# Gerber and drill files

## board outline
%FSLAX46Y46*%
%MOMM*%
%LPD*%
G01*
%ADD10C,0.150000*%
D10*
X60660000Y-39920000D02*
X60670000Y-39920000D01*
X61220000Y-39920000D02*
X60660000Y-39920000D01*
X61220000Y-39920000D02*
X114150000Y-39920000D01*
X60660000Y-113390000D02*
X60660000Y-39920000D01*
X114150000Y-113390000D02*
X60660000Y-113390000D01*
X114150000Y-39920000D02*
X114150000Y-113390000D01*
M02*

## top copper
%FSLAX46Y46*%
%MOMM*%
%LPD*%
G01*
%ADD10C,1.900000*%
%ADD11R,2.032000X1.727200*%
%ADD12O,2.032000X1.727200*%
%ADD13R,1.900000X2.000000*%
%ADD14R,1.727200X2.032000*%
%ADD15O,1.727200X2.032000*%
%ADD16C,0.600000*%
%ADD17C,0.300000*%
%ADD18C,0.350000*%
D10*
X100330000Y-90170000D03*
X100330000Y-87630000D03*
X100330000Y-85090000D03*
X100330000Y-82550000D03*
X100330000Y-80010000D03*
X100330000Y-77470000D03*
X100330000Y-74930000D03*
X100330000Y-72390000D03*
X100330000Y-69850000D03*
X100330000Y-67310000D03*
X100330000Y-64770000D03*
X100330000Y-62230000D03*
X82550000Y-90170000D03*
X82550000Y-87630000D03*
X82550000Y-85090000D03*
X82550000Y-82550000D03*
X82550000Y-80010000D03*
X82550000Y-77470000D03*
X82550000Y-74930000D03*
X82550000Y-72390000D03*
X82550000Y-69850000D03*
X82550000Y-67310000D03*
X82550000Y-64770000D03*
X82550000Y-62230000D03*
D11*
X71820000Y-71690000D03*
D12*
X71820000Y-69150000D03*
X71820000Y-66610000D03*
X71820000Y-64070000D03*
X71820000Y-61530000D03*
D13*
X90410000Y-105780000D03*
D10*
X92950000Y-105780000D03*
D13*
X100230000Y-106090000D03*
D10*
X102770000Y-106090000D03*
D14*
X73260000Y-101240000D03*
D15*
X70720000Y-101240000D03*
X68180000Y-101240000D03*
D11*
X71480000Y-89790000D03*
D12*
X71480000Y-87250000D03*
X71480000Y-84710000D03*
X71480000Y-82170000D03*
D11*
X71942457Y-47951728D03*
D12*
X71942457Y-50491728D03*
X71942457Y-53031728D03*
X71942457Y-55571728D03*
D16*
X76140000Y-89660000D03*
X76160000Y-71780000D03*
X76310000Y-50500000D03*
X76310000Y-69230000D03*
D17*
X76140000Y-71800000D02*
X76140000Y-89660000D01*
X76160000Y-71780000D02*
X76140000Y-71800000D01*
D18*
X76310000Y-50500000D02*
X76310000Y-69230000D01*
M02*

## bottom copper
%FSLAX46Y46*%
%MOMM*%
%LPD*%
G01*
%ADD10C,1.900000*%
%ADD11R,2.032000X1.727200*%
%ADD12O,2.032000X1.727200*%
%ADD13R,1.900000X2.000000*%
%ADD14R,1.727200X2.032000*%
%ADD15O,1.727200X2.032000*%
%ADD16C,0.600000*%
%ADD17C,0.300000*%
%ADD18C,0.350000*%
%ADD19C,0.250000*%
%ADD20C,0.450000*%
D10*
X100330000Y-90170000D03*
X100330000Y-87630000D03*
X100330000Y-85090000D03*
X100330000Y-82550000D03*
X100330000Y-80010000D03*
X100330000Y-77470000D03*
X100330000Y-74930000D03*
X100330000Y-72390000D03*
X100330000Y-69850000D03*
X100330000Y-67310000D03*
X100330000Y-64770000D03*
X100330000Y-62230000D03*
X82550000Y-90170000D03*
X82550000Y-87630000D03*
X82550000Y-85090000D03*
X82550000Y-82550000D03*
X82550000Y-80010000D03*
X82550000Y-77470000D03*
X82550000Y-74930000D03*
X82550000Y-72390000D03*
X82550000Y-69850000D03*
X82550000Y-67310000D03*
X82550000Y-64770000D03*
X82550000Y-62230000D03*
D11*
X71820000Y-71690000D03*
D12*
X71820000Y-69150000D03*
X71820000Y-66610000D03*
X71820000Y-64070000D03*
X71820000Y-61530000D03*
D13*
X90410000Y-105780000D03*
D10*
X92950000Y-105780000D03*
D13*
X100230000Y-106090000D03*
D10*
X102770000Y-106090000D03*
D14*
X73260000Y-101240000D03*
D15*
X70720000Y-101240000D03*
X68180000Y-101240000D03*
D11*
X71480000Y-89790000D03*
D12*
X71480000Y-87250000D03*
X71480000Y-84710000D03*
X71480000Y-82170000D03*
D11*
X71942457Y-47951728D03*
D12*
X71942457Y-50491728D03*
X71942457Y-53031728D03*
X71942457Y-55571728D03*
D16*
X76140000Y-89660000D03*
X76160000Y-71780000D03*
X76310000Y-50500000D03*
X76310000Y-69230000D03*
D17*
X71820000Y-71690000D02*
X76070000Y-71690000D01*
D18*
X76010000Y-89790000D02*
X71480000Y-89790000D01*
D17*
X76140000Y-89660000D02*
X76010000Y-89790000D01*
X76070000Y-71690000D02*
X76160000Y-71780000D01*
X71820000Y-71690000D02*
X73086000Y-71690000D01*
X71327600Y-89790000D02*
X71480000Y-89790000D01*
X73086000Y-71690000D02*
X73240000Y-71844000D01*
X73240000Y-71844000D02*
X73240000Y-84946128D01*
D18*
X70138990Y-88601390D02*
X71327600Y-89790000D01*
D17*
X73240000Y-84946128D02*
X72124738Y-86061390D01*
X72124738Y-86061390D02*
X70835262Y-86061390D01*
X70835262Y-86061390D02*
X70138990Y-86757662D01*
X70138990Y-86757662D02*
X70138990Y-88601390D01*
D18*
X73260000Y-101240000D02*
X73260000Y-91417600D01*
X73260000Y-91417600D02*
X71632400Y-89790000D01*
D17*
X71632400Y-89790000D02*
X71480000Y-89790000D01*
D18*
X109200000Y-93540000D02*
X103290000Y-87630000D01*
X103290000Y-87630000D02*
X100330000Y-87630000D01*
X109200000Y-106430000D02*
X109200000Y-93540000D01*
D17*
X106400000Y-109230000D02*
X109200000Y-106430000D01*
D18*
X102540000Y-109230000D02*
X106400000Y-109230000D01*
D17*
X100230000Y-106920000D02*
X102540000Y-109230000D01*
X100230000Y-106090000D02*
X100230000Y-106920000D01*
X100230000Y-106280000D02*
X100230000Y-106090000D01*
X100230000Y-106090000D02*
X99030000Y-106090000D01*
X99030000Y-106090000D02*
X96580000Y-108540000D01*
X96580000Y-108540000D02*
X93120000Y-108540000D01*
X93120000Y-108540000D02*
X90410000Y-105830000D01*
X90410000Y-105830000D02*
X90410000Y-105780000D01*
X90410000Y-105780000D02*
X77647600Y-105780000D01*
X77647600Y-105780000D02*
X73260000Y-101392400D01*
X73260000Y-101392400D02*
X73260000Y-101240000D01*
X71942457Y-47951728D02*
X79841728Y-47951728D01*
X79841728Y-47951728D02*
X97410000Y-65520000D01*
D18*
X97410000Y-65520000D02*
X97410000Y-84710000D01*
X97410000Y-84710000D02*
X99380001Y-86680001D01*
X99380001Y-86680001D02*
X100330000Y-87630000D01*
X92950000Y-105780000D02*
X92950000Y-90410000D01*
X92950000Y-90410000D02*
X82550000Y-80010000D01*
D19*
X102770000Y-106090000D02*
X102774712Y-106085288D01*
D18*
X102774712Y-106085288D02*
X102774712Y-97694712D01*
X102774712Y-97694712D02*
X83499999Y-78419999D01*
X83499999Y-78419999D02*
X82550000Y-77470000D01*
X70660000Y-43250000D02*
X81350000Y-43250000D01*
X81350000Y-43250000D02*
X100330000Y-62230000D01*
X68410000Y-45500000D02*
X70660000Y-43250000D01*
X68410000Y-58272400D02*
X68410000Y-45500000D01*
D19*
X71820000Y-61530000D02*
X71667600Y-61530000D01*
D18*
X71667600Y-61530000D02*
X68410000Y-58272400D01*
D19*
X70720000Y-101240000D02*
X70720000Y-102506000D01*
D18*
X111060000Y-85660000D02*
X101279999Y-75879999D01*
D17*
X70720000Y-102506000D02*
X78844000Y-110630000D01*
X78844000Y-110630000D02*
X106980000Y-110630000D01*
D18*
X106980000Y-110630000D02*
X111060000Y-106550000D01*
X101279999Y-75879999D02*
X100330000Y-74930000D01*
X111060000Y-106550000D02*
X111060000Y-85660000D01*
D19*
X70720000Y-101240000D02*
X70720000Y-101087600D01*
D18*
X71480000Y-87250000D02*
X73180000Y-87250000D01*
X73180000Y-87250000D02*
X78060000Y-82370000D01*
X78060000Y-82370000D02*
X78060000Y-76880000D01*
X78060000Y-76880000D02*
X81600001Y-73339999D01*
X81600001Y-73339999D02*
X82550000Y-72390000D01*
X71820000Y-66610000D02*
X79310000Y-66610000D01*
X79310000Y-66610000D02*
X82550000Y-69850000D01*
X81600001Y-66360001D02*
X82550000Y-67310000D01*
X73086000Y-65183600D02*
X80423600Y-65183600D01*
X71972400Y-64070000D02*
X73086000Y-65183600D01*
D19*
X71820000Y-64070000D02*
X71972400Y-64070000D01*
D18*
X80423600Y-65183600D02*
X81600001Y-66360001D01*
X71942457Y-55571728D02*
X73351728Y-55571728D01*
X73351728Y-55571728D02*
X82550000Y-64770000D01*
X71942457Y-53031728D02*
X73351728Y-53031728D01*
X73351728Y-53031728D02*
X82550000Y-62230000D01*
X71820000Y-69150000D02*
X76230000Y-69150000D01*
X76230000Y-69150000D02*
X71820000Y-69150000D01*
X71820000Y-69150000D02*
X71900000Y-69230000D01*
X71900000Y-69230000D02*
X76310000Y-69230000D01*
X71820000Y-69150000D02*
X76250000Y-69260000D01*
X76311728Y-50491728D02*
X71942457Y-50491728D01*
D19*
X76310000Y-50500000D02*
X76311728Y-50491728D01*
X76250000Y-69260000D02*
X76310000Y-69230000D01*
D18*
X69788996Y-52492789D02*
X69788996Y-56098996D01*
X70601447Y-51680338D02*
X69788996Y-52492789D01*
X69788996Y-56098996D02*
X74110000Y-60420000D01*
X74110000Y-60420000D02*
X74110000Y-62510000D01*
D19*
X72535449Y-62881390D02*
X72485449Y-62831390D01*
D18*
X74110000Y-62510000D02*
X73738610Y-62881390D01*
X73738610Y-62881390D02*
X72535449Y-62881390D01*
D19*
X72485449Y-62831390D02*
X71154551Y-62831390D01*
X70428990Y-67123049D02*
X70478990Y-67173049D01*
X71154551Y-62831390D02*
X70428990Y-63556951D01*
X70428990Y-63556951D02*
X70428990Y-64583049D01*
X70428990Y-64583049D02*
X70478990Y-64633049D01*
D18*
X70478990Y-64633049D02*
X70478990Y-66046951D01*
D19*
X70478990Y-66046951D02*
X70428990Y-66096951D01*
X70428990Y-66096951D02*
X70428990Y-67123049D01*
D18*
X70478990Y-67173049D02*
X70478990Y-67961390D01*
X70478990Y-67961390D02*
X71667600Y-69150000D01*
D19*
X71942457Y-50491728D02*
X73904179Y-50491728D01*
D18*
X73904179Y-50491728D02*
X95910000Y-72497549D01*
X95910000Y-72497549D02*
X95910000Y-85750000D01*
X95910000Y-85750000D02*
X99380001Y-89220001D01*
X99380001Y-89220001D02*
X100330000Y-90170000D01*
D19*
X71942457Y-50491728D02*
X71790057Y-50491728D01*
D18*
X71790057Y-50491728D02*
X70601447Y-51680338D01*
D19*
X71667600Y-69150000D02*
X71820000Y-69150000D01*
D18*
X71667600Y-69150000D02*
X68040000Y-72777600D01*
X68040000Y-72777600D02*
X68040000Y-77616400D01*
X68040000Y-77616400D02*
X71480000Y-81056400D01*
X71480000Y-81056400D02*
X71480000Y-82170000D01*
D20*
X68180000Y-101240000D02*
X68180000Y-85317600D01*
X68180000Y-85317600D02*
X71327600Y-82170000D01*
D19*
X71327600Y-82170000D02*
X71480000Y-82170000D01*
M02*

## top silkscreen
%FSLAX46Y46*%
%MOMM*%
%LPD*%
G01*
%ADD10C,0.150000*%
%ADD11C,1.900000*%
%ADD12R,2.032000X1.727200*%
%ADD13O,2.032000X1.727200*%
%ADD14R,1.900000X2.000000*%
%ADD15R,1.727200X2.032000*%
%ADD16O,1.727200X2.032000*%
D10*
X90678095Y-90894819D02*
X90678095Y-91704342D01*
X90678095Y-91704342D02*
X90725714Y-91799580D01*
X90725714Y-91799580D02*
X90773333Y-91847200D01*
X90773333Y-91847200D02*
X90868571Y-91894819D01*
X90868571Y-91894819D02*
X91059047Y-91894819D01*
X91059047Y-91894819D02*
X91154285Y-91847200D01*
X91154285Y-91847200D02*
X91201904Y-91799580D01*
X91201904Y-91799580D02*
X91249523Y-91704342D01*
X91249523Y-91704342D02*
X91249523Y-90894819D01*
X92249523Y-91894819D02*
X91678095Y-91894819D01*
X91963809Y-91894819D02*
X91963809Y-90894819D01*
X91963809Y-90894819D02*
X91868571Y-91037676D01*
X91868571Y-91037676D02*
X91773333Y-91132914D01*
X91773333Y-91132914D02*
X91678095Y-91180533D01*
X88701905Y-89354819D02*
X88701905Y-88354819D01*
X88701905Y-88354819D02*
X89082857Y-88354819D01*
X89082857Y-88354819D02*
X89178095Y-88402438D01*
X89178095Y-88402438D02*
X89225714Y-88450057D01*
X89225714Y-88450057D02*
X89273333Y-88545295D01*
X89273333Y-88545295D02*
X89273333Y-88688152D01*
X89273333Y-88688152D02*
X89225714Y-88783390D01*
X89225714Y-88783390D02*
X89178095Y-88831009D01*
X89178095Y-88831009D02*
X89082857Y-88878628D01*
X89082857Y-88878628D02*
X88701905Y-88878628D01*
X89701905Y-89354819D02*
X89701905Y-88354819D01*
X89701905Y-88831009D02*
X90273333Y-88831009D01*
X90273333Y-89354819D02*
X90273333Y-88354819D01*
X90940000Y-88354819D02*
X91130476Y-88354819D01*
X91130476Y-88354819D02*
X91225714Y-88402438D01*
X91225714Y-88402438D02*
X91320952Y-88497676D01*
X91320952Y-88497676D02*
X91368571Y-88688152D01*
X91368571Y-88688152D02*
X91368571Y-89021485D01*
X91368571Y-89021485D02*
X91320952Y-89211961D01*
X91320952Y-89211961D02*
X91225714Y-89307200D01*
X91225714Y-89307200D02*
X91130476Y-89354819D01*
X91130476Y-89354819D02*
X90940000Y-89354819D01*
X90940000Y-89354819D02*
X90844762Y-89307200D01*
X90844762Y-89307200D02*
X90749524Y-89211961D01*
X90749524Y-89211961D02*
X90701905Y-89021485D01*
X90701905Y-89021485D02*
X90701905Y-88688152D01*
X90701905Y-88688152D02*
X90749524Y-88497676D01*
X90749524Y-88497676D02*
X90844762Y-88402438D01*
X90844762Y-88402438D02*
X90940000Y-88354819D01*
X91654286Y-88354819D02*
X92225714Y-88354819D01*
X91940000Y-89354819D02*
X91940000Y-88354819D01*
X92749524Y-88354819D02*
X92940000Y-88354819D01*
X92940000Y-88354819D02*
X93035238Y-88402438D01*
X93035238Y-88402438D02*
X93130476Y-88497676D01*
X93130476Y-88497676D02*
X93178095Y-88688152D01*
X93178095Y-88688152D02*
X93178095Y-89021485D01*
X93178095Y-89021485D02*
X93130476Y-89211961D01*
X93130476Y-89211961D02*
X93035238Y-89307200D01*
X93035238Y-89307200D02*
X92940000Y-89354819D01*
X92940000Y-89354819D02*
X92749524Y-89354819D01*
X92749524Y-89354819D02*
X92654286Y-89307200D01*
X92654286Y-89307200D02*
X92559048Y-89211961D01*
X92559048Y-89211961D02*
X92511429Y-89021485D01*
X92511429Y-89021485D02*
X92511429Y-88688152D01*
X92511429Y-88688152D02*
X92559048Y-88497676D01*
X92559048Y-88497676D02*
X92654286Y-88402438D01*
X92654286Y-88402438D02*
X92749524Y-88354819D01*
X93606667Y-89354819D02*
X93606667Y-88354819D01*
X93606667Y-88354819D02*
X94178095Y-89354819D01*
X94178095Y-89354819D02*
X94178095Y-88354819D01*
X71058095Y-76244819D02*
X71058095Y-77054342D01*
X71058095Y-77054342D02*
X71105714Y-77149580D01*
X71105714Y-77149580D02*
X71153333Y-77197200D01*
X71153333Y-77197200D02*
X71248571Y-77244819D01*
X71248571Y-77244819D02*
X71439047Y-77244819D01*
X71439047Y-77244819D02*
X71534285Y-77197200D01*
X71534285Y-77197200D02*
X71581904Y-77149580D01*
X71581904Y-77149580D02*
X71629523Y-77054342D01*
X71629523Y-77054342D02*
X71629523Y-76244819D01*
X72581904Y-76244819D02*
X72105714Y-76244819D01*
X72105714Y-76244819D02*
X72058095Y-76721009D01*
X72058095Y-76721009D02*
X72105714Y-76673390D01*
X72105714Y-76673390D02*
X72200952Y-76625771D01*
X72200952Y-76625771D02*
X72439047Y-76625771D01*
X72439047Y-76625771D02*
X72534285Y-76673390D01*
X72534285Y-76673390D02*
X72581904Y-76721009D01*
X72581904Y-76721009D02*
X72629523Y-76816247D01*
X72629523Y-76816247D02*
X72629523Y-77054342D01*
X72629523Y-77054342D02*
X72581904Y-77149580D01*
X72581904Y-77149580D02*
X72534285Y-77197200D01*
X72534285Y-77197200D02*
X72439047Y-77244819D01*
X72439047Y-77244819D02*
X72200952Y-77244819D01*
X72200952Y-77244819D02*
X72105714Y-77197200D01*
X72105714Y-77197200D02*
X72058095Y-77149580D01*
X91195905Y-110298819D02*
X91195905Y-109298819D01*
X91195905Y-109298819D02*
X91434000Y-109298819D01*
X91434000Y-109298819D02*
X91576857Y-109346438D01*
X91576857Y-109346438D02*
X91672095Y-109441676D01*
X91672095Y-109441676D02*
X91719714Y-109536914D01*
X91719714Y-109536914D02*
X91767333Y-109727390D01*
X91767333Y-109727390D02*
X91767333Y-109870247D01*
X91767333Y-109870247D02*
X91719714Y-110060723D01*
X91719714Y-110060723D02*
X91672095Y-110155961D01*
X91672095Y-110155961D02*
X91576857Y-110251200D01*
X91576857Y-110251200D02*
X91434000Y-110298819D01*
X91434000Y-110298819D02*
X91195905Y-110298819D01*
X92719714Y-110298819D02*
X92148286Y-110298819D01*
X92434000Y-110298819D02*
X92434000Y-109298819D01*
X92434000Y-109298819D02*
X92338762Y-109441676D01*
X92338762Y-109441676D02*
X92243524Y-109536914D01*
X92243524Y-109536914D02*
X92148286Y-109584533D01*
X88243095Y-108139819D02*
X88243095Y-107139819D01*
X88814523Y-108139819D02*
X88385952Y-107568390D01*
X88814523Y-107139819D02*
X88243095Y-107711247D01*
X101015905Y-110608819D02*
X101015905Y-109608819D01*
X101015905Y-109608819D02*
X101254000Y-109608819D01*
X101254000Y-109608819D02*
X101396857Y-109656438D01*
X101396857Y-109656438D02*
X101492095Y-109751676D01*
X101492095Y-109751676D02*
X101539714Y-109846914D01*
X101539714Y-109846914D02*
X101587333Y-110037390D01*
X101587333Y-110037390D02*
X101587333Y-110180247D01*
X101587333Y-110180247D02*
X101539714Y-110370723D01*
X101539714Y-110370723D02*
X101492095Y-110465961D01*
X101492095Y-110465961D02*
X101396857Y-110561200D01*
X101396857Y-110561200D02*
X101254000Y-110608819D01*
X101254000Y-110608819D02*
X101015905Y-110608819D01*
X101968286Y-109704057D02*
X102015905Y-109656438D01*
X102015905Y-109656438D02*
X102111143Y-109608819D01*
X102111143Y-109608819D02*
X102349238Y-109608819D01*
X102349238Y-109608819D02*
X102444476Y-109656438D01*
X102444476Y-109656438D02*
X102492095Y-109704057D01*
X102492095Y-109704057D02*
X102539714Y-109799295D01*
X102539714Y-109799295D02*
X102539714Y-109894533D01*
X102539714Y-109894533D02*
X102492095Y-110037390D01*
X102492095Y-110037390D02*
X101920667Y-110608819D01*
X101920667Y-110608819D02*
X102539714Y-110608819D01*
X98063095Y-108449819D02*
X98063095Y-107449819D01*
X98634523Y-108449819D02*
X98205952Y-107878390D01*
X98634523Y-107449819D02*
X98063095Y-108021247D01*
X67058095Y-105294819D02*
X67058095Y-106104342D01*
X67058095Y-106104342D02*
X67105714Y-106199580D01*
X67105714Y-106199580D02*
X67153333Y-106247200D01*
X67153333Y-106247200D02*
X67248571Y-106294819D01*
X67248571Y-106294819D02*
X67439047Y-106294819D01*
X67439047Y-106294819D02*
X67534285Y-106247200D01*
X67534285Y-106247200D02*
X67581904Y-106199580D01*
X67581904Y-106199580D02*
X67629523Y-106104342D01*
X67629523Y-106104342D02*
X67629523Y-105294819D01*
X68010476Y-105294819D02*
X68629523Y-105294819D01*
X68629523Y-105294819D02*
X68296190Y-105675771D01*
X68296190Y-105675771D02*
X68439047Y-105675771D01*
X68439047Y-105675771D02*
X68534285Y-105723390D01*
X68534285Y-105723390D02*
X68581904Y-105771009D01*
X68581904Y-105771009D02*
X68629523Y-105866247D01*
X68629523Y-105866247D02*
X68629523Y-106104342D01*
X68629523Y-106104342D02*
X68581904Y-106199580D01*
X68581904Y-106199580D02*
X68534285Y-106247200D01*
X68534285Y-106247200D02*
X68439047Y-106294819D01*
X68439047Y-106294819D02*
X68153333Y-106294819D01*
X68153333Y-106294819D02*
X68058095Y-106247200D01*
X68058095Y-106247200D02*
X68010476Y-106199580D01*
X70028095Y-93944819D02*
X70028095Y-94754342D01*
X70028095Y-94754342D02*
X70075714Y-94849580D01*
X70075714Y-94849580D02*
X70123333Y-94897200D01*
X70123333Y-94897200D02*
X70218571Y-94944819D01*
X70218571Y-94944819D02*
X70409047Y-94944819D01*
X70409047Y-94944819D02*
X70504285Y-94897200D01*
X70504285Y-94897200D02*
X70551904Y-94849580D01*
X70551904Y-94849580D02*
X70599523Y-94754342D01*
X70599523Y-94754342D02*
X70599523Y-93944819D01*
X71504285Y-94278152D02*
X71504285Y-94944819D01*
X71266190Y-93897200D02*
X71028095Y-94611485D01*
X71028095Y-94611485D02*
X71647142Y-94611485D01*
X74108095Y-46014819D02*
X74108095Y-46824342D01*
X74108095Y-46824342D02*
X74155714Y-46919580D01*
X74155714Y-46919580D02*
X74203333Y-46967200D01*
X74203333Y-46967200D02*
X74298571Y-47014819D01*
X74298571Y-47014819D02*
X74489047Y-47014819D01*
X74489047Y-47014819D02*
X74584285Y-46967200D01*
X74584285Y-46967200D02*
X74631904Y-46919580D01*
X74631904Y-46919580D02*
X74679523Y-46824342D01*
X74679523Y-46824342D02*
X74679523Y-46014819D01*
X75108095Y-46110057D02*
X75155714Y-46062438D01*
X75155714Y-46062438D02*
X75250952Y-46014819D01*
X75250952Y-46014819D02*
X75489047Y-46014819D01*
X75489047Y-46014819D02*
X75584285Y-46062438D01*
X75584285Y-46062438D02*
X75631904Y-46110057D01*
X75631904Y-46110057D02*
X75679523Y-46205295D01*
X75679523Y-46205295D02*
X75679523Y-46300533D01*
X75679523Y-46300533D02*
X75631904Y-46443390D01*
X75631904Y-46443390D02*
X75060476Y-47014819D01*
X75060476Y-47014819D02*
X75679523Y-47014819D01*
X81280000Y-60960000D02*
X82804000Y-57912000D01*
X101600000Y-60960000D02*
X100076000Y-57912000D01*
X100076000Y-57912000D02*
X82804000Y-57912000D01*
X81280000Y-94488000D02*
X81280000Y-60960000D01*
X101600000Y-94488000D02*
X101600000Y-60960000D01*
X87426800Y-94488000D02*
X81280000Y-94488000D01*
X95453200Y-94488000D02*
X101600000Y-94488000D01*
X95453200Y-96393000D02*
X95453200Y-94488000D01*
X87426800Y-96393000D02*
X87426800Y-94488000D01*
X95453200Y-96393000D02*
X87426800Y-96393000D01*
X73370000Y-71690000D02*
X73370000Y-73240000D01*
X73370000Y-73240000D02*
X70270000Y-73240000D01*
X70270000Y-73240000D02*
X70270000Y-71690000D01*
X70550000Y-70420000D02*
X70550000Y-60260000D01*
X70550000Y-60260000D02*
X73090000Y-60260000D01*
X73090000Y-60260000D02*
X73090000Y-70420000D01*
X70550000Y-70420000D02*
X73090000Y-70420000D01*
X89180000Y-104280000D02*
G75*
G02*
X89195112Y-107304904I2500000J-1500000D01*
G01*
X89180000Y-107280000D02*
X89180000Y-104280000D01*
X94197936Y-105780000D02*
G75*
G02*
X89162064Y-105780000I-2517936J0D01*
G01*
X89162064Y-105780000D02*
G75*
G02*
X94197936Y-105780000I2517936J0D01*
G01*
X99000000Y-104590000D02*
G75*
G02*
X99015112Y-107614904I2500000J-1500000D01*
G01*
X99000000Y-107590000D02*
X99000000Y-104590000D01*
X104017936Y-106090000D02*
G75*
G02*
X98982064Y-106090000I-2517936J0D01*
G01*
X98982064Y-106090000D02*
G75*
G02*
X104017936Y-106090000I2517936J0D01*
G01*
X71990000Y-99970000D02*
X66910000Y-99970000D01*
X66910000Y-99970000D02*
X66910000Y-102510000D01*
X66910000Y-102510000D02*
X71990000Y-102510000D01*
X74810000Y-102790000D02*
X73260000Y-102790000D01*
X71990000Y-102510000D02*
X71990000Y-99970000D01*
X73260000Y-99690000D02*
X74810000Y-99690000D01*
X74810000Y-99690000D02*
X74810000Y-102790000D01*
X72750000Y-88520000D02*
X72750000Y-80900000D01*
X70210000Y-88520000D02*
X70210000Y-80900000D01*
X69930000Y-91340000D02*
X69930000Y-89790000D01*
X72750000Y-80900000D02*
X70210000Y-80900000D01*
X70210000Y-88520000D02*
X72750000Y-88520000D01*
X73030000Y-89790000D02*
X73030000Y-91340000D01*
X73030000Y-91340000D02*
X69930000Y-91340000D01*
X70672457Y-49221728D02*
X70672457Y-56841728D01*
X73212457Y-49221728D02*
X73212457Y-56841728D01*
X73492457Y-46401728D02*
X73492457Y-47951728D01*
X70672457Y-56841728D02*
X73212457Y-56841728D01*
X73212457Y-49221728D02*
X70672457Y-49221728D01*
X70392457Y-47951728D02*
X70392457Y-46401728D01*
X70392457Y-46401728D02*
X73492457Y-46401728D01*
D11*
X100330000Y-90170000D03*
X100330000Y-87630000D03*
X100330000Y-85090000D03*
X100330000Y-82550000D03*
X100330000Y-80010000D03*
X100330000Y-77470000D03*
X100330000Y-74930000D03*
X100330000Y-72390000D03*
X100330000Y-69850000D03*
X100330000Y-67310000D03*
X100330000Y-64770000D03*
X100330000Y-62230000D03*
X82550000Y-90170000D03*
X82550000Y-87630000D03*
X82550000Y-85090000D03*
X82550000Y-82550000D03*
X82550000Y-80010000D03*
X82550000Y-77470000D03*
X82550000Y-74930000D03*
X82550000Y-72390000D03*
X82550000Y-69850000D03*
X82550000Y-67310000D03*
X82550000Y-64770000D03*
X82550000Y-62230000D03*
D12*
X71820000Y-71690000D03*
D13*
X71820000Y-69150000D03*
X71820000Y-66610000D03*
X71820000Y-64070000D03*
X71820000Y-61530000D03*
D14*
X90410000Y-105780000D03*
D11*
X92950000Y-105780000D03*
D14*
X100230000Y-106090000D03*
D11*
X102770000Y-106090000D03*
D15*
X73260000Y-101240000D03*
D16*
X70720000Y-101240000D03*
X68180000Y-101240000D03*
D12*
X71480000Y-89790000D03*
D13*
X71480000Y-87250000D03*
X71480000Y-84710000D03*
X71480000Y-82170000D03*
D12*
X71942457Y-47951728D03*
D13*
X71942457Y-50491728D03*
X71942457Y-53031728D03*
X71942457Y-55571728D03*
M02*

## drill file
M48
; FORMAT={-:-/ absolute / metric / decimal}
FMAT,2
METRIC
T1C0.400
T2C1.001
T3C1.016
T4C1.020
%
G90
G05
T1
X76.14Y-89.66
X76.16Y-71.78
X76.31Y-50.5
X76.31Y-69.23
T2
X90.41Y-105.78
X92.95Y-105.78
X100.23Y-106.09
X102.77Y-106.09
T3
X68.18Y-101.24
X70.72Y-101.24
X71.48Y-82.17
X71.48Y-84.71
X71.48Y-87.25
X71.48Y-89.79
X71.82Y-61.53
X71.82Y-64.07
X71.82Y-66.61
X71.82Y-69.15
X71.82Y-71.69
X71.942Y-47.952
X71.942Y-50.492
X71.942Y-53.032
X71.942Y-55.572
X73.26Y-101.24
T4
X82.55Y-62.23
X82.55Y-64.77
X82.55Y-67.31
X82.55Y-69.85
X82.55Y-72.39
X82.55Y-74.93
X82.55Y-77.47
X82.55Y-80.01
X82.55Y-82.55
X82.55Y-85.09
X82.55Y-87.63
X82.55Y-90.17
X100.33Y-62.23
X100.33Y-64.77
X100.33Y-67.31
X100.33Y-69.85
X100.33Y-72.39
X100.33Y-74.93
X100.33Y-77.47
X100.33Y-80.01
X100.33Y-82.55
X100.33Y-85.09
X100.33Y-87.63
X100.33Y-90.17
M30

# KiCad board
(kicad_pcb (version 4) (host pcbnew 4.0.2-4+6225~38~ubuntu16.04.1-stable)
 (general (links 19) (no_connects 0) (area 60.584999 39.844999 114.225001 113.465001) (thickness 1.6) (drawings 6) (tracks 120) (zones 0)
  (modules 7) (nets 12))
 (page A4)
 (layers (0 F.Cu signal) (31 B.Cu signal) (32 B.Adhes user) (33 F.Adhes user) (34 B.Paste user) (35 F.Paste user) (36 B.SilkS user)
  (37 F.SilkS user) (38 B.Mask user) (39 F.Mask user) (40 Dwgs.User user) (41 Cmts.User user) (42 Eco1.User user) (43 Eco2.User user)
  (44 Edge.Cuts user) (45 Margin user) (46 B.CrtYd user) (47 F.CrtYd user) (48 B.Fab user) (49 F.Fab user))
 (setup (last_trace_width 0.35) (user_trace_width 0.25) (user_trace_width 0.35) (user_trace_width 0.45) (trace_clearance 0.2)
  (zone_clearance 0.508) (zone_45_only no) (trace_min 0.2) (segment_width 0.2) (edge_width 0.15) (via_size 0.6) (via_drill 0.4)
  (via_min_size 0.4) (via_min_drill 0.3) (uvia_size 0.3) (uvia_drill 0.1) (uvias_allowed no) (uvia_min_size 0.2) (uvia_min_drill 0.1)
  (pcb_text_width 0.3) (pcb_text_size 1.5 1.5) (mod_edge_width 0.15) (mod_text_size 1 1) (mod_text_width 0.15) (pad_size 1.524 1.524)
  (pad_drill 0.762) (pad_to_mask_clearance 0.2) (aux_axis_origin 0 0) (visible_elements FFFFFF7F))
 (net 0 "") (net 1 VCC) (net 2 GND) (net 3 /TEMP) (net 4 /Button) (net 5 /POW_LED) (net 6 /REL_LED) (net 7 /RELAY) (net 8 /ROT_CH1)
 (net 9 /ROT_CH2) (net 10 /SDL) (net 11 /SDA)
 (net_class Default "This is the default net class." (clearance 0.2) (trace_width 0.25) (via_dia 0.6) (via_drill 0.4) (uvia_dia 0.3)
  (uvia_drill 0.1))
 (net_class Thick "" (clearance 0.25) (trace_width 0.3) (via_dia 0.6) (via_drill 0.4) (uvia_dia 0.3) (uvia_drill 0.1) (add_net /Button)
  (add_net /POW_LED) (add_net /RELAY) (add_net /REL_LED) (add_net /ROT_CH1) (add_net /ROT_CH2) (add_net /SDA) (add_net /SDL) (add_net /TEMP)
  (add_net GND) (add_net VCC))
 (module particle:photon (layer F.Cu) (at 91.44 74.93 180)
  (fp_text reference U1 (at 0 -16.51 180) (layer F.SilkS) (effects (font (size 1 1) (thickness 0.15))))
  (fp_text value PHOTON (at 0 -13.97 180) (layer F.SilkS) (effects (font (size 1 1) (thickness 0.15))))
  (fp_line (start 10.16 13.97) (end 8.636 17.018) (layer F.SilkS) (width 0.15))
  (fp_line (start -10.16 13.97) (end -8.636 17.018) (layer F.SilkS) (width 0.15))
  (fp_line (start -8.636 17.018) (end 8.636 17.018) (layer F.SilkS) (width 0.15))
  (fp_line (start 10.16 -19.558) (end 10.16 13.97) (layer F.SilkS) (width 0.15))
  (fp_line (start -10.16 -19.558) (end -10.16 13.97) (layer F.SilkS) (width 0.15))
  (fp_line (start 4.0132 -19.558) (end 10.16 -19.558) (layer F.SilkS) (width 0.15))
  (fp_line (start -4.0132 -19.558) (end -10.16 -19.558) (layer F.SilkS) (width 0.15))
  (fp_line (start -4.0132 -21.463) (end -4.0132 -19.558) (layer F.SilkS) (width 0.15))
  (fp_line (start 4.0132 -21.463) (end 4.0132 -19.558) (layer F.SilkS) (width 0.15))
  (fp_line (start -4.0132 -21.463) (end 4.0132 -21.463) (layer F.SilkS) (width 0.15))
  (pad 1 thru_hole circle (at -8.89 -15.24 180) (size 1.9 1.9) (drill 1.02) (layers *.Cu *.Mask F.SilkS) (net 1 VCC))
  (pad 2 thru_hole circle (at -8.89 -12.7 180) (size 1.9 1.9) (drill 1.02) (layers *.Cu *.Mask F.SilkS) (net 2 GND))
  (pad 3 thru_hole circle (at -8.89 -10.16 180) (size 1.9 1.9) (drill 1.02) (layers *.Cu *.Mask F.SilkS))
  (pad 4 thru_hole circle (at -8.89 -7.62 180) (size 1.9 1.9) (drill 1.02) (layers *.Cu *.Mask F.SilkS))
  (pad 5 thru_hole circle (at -8.89 -5.08 180) (size 1.9 1.9) (drill 1.02) (layers *.Cu *.Mask F.SilkS))
  (pad 6 thru_hole circle (at -8.89 -2.54 180) (size 1.9 1.9) (drill 1.02) (layers *.Cu *.Mask F.SilkS))
  (pad 7 thru_hole circle (at -8.89 0 180) (size 1.9 1.9) (drill 1.02) (layers *.Cu *.Mask F.SilkS) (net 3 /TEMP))
  (pad 8 thru_hole circle (at -8.89 2.54 180) (size 1.9 1.9) (drill 1.02) (layers *.Cu *.Mask F.SilkS))
  (pad 9 thru_hole circle (at -8.89 5.08 180) (size 1.9 1.9) (drill 1.02) (layers *.Cu *.Mask F.SilkS))
  (pad 10 thru_hole circle (at -8.89 7.62 180) (size 1.9 1.9) (drill 1.02) (layers *.Cu *.Mask F.SilkS))
  (pad 11 thru_hole circle (at -8.89 10.16 180) (size 1.9 1.9) (drill 1.02) (layers *.Cu *.Mask F.SilkS))
  (pad 12 thru_hole circle (at -8.89 12.7 180) (size 1.9 1.9) (drill 1.02) (layers *.Cu *.Mask F.SilkS) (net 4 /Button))
  (pad 24 thru_hole circle (at 8.89 -15.24 180) (size 1.9 1.9) (drill 1.02) (layers *.Cu *.Mask F.SilkS))
  (pad 23 thru_hole circle (at 8.89 -12.7 180) (size 1.9 1.9) (drill 1.02) (layers *.Cu *.Mask F.SilkS))
  (pad 22 thru_hole circle (at 8.89 -10.16 180) (size 1.9 1.9) (drill 1.02) (layers *.Cu *.Mask F.SilkS))
  (pad 21 thru_hole circle (at 8.89 -7.62 180) (size 1.9 1.9) (drill 1.02) (layers *.Cu *.Mask F.SilkS))
  (pad 20 thru_hole circle (at 8.89 -5.08 180) (size 1.9 1.9) (drill 1.02) (layers *.Cu *.Mask F.SilkS) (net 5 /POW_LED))
  (pad 19 thru_hole circle (at 8.89 -2.54 180) (size 1.9 1.9) (drill 1.02) (layers *.Cu *.Mask F.SilkS) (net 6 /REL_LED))
  (pad 18 thru_hole circle (at 8.89 0 180) (size 1.9 1.9) (drill 1.02) (layers *.Cu *.Mask F.SilkS))
  (pad 17 thru_hole circle (at 8.89 2.54 180) (size 1.9 1.9) (drill 1.02) (layers *.Cu *.Mask F.SilkS) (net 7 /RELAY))
  (pad 16 thru_hole circle (at 8.89 5.08 180) (size 1.9 1.9) (drill 1.02) (layers *.Cu *.Mask F.SilkS) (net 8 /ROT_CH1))
  (pad 15 thru_hole circle (at 8.89 7.62 180) (size 1.9 1.9) (drill 1.02) (layers *.Cu *.Mask F.SilkS) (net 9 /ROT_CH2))
  (pad 14 thru_hole circle (at 8.89 10.16 180) (size 1.9 1.9) (drill 1.02) (layers *.Cu *.Mask F.SilkS) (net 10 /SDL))
  (pad 13 thru_hole circle (at 8.89 12.7 180) (size 1.9 1.9) (drill 1.02) (layers *.Cu *.Mask F.SilkS) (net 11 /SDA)))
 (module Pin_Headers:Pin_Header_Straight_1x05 (layer F.Cu) (at 71.82 71.69 180)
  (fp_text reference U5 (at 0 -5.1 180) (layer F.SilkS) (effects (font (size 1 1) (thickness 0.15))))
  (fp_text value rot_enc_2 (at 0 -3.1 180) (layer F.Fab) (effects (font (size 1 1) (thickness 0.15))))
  (fp_line (start -1.55 0) (end -1.55 -1.55) (layer F.SilkS) (width 0.15))
  (fp_line (start -1.55 -1.55) (end 1.55 -1.55) (layer F.SilkS) (width 0.15))
  (fp_line (start 1.55 -1.55) (end 1.55 0) (layer F.SilkS) (width 0.15))
  (fp_line (start 1.27 1.27) (end 1.27 11.43) (layer F.SilkS) (width 0.15))
  (fp_line (start 1.27 11.43) (end -1.27 11.43) (layer F.SilkS) (width 0.15))
  (fp_line (start -1.27 11.43) (end -1.27 1.27) (layer F.SilkS) (width 0.15))
  (fp_line (start 1.27 1.27) (end -1.27 1.27) (layer F.SilkS) (width 0.15))
  (pad 1 thru_hole rect (at 0 0 180) (size 2.032 1.7272) (drill 1.016) (layers *.Cu *.Mask F.SilkS) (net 2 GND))
  (pad 2 thru_hole oval (at 0 2.54 180) (size 2.032 1.7272) (drill 1.016) (layers *.Cu *.Mask F.SilkS) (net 1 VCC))
  (pad 3 thru_hole oval (at 0 5.08 180) (size 2.032 1.7272) (drill 1.016) (layers *.Cu *.Mask F.SilkS) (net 8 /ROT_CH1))
  (pad 4 thru_hole oval (at 0 7.62 180) (size 2.032 1.7272) (drill 1.016) (layers *.Cu *.Mask F.SilkS) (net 9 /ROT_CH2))
  (pad 5 thru_hole oval (at 0 10.16 180) (size 2.032 1.7272) (drill 1.016) (layers *.Cu *.Mask F.SilkS) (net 4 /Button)))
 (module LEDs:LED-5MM (layer F.Cu) (at 90.41 105.78)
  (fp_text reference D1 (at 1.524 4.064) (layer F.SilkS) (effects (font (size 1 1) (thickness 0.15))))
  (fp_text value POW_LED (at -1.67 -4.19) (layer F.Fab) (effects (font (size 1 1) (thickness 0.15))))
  (fp_arc (start 1.27 0) (end -1.23 -1.5) (angle 297.5) (layer F.SilkS) (width 0.15))
  (fp_line (start -1.23 1.5) (end -1.23 -1.5) (layer F.SilkS) (width 0.15))
  (fp_circle (center 1.27 0) (end 0.97 -2.5) (layer F.SilkS) (width 0.15))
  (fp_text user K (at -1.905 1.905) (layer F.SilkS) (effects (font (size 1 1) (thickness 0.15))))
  (pad 1 thru_hole rect (at 0 0 90) (size 2 1.9) (drill 1.00076) (layers *.Cu *.Mask F.SilkS) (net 2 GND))
  (pad 2 thru_hole circle (at 2.54 0) (size 1.9 1.9) (drill 1.00076) (layers *.Cu *.Mask F.SilkS) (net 5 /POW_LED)))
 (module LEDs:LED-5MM (layer F.Cu) (at 100.23 106.09)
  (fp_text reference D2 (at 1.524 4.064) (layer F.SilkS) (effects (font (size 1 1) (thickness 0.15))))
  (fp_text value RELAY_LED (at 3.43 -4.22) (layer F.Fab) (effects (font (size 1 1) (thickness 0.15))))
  (fp_arc (start 1.27 0) (end -1.23 -1.5) (angle 297.5) (layer F.SilkS) (width 0.15))
  (fp_line (start -1.23 1.5) (end -1.23 -1.5) (layer F.SilkS) (width 0.15))
  (fp_circle (center 1.27 0) (end 0.97 -2.5) (layer F.SilkS) (width 0.15))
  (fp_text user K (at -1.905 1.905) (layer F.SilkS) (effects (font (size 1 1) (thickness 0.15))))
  (pad 1 thru_hole rect (at 0 0 90) (size 2 1.9) (drill 1.00076) (layers *.Cu *.Mask F.SilkS) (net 2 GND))
  (pad 2 thru_hole circle (at 2.54 0) (size 1.9 1.9) (drill 1.00076) (layers *.Cu *.Mask F.SilkS) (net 6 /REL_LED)))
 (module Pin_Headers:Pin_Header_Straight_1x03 (layer F.Cu) (at 73.26 101.24 270)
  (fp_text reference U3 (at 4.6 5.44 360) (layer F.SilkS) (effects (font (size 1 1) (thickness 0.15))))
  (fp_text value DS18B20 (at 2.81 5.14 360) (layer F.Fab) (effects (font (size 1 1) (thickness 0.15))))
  (fp_line (start -1.27 1.27) (end -1.27 6.35) (layer F.SilkS) (width 0.15))
  (fp_line (start -1.27 6.35) (end 1.27 6.35) (layer F.SilkS) (width 0.15))
  (fp_line (start 1.27 6.35) (end 1.27 1.27) (layer F.SilkS) (width 0.15))
  (fp_line (start 1.55 -1.55) (end 1.55 0) (layer F.SilkS) (width 0.15))
  (fp_line (start 1.27 1.27) (end -1.27 1.27) (layer F.SilkS) (width 0.15))
  (fp_line (start -1.55 0) (end -1.55 -1.55) (layer F.SilkS) (width 0.15))
  (fp_line (start -1.55 -1.55) (end 1.55 -1.55) (layer F.SilkS) (width 0.15))
  (pad 1 thru_hole rect (at 0 0 270) (size 2.032 1.7272) (drill 1.016) (layers *.Cu *.Mask F.SilkS) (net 2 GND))
  (pad 2 thru_hole oval (at 0 2.54 270) (size 2.032 1.7272) (drill 1.016) (layers *.Cu *.Mask F.SilkS) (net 3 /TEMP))
  (pad 3 thru_hole oval (at 0 5.08 270) (size 2.032 1.7272) (drill 1.016) (layers *.Cu *.Mask F.SilkS) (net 1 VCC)))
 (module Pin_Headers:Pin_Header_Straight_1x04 (layer F.Cu) (at 71.48 89.79 180)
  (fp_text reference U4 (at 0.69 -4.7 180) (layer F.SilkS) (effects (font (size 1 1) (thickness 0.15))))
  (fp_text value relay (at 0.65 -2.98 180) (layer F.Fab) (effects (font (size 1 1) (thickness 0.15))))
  (fp_line (start -1.27 1.27) (end -1.27 8.89) (layer F.SilkS) (width 0.15))
  (fp_line (start 1.27 1.27) (end 1.27 8.89) (layer F.SilkS) (width 0.15))
  (fp_line (start 1.55 -1.55) (end 1.55 0) (layer F.SilkS) (width 0.15))
  (fp_line (start -1.27 8.89) (end 1.27 8.89) (layer F.SilkS) (width 0.15))
  (fp_line (start 1.27 1.27) (end -1.27 1.27) (layer F.SilkS) (width 0.15))
  (fp_line (start -1.55 0) (end -1.55 -1.55) (layer F.SilkS) (width 0.15))
  (fp_line (start -1.55 -1.55) (end 1.55 -1.55) (layer F.SilkS) (width 0.15))
  (pad 1 thru_hole rect (at 0 0 180) (size 2.032 1.7272) (drill 1.016) (layers *.Cu *.Mask F.SilkS) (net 2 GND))
  (pad 2 thru_hole oval (at 0 2.54 180) (size 2.032 1.7272) (drill 1.016) (layers *.Cu *.Mask F.SilkS) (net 7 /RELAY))
  (pad 3 thru_hole oval (at 0 5.08 180) (size 2.032 1.7272) (drill 1.016) (layers *.Cu *.Mask F.SilkS))
  (pad 4 thru_hole oval (at 0 7.62 180) (size 2.032 1.7272) (drill 1.016) (layers *.Cu *.Mask F.SilkS) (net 1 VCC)))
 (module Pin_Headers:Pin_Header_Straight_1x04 (layer F.Cu) (at 71.942457 47.951728)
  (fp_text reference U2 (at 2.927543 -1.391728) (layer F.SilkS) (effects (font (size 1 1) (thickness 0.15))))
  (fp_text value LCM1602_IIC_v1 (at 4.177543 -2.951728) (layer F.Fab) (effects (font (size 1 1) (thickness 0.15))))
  (fp_line (start -1.27 1.27) (end -1.27 8.89) (layer F.SilkS) (width 0.15))
  (fp_line (start 1.27 1.27) (end 1.27 8.89) (layer F.SilkS) (width 0.15))
  (fp_line (start 1.55 -1.55) (end 1.55 0) (layer F.SilkS) (width 0.15))
  (fp_line (start -1.27 8.89) (end 1.27 8.89) (layer F.SilkS) (width 0.15))
  (fp_line (start 1.27 1.27) (end -1.27 1.27) (layer F.SilkS) (width 0.15))
  (fp_line (start -1.55 0) (end -1.55 -1.55) (layer F.SilkS) (width 0.15))
  (fp_line (start -1.55 -1.55) (end 1.55 -1.55) (layer F.SilkS) (width 0.15))
  (pad 1 thru_hole rect (at 0 0) (size 2.032 1.7272) (drill 1.016) (layers *.Cu *.Mask F.SilkS) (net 2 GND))
  (pad 2 thru_hole oval (at 0 2.54) (size 2.032 1.7272) (drill 1.016) (layers *.Cu *.Mask F.SilkS) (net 1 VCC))
  (pad 3 thru_hole oval (at 0 5.08) (size 2.032 1.7272) (drill 1.016) (layers *.Cu *.Mask F.SilkS) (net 11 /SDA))
  (pad 4 thru_hole oval (at 0 7.62) (size 2.032 1.7272) (drill 1.016) (layers *.Cu *.Mask F.SilkS) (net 10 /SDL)))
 (gr_line (start 60.66 39.92) (end 60.67 39.92) (angle 90) (layer Edge.Cuts) (width 0.15))
 (gr_line (start 61.22 39.92) (end 60.66 39.92) (angle 90) (layer Edge.Cuts) (width 0.15))
 (gr_line (start 61.22 39.92) (end 114.15 39.92) (angle 90) (layer Edge.Cuts) (width 0.15))
 (gr_line (start 60.66 113.39) (end 60.66 39.92) (angle 90) (layer Edge.Cuts) (width 0.15))
 (gr_line (start 114.15 113.39) (end 60.66 113.39) (angle 90) (layer Edge.Cuts) (width 0.15))
 (gr_line (start 114.15 39.92) (end 114.15 113.39) (angle 90) (layer Edge.Cuts) (width 0.15))
 (segment (start 71.82 71.69) (end 76.07 71.69) (width 0.3) (layer B.Cu) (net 2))
 (segment (start 76.01 89.79) (end 71.48 89.79) (width 0.35) (layer B.Cu) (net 2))
 (segment (start 76.14 89.66) (end 76.01 89.79) (width 0.3) (layer B.Cu) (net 2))
 (via (at 76.14 89.66) (size 0.6) (drill 0.4) (layers F.Cu B.Cu) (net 2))
 (segment (start 76.14 71.8) (end 76.14 89.66) (width 0.3) (layer F.Cu) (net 2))
 (segment (start 76.16 71.78) (end 76.14 71.8) (width 0.3) (layer F.Cu) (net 2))
 (via (at 76.16 71.78) (size 0.6) (drill 0.4) (layers F.Cu B.Cu) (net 2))
 (segment (start 76.07 71.69) (end 76.16 71.78) (width 0.3) (layer B.Cu) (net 2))
 (segment (start 71.82 71.69) (end 73.086 71.69) (width 0.3) (layer B.Cu) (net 2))
 (segment (start 71.3276 89.79) (end 71.48 89.79) (width 0.3) (layer B.Cu) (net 2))
 (segment (start 73.086 71.69) (end 73.24 71.844) (width 0.3) (layer B.Cu) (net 2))
 (segment (start 73.24 71.844) (end 73.24 84.946128) (width 0.3) (layer B.Cu) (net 2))
 (segment (start 70.13899 88.60139) (end 71.3276 89.79) (width 0.35) (layer B.Cu) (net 2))
 (segment (start 73.24 84.946128) (end 72.124738 86.06139) (width 0.3) (layer B.Cu) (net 2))
 (segment (start 72.124738 86.06139) (end 70.835262 86.06139) (width 0.3) (layer B.Cu) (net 2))
 (segment (start 70.835262 86.06139) (end 70.13899 86.757662) (width 0.3) (layer B.Cu) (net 2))
 (segment (start 70.13899 86.757662) (end 70.13899 88.60139) (width 0.3) (layer B.Cu) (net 2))
 (segment (start 73.26 101.24) (end 73.26 91.4176) (width 0.35) (layer B.Cu) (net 2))
 (segment (start 73.26 91.4176) (end 71.6324 89.79) (width 0.35) (layer B.Cu) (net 2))
 (segment (start 71.6324 89.79) (end 71.48 89.79) (width 0.3) (layer B.Cu) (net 2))
 (segment (start 109.2 93.54) (end 103.29 87.63) (width 0.35) (layer B.Cu) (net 2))
 (segment (start 103.29 87.63) (end 100.33 87.63) (width 0.35) (layer B.Cu) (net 2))
 (segment (start 109.2 106.43) (end 109.2 93.54) (width 0.35) (layer B.Cu) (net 2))
 (segment (start 106.4 109.23) (end 109.2 106.43) (width 0.3) (layer B.Cu) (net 2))
 (segment (start 102.54 109.23) (end 106.4 109.23) (width 0.35) (layer B.Cu) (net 2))
 (segment (start 100.23 106.92) (end 102.54 109.23) (width 0.3) (layer B.Cu) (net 2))
 (segment (start 100.23 106.09) (end 100.23 106.92) (width 0.3) (layer B.Cu) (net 2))
 (segment (start 100.23 106.28) (end 100.23 106.09) (width 0.3) (layer B.Cu) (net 2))
 (segment (start 100.23 106.09) (end 99.03 106.09) (width 0.3) (layer B.Cu) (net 2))
 (segment (start 99.03 106.09) (end 96.58 108.54) (width 0.3) (layer B.Cu) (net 2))
 (segment (start 96.58 108.54) (end 93.12 108.54) (width 0.3) (layer B.Cu) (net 2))
 (segment (start 93.12 108.54) (end 90.41 105.83) (width 0.3) (layer B.Cu) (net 2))
 (segment (start 90.41 105.83) (end 90.41 105.78) (width 0.3) (layer B.Cu) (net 2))
 (segment (start 90.41 105.78) (end 77.6476 105.78) (width 0.3) (layer B.Cu) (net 2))
 (segment (start 77.6476 105.78) (end 73.26 101.3924) (width 0.3) (layer B.Cu) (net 2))
 (segment (start 73.26 101.3924) (end 73.26 101.24) (width 0.3) (layer B.Cu) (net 2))
 (segment (start 71.942457 47.951728) (end 79.841728 47.951728) (width 0.3) (layer B.Cu) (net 2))
 (segment (start 79.841728 47.951728) (end 97.41 65.52) (width 0.3) (layer B.Cu) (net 2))
 (segment (start 97.41 65.52) (end 97.41 84.71) (width 0.35) (layer B.Cu) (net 2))
 (segment (start 97.41 84.71) (end 99.380001 86.680001) (width 0.35) (layer B.Cu) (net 2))
 (segment (start 99.380001 86.680001) (end 100.33 87.63) (width 0.35) (layer B.Cu) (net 2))
 (segment (start 92.95 105.78) (end 92.95 90.41) (width 0.35) (layer B.Cu) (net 5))
 (segment (start 92.95 90.41) (end 82.55 80.01) (width 0.35) (layer B.Cu) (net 5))
 (segment (start 102.77 106.09) (end 102.774712 106.085288) (width 0.25) (layer B.Cu) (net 6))
 (segment (start 102.774712 106.085288) (end 102.774712 97.694712) (width 0.35) (layer B.Cu) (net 6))
 (segment (start 102.774712 97.694712) (end 83.499999 78.419999) (width 0.35) (layer B.Cu) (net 6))
 (segment (start 83.499999 78.419999) (end 82.55 77.47) (width 0.35) (layer B.Cu) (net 6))
 (segment (start 70.66 43.25) (end 81.35 43.25) (width 0.35) (layer B.Cu) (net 4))
 (segment (start 81.35 43.25) (end 100.33 62.23) (width 0.35) (layer B.Cu) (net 4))
 (segment (start 68.41 45.5) (end 70.66 43.25) (width 0.35) (layer B.Cu) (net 4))
 (segment (start 68.41 58.2724) (end 68.41 45.5) (width 0.35) (layer B.Cu) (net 4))
 (segment (start 71.82 61.53) (end 71.6676 61.53) (width 0.25) (layer B.Cu) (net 4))
 (segment (start 71.6676 61.53) (end 68.41 58.2724) (width 0.35) (layer B.Cu) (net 4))
 (segment (start 70.72 101.24) (end 70.72 102.506) (width 0.25) (layer B.Cu) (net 3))
 (segment (start 111.06 85.66) (end 101.279999 75.879999) (width 0.35) (layer B.Cu) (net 3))
 (segment (start 70.72 102.506) (end 78.844 110.63) (width 0.3) (layer B.Cu) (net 3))
 (segment (start 78.844 110.63) (end 106.98 110.63) (width 0.3) (layer B.Cu) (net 3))
 (segment (start 106.98 110.63) (end 111.06 106.55) (width 0.35) (layer B.Cu) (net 3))
 (segment (start 101.279999 75.879999) (end 100.33 74.93) (width 0.35) (layer B.Cu) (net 3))
 (segment (start 111.06 106.55) (end 111.06 85.66) (width 0.35) (layer B.Cu) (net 3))
 (segment (start 70.72 101.24) (end 70.72 101.0876) (width 0.25) (layer B.Cu) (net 3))
 (segment (start 71.48 87.25) (end 73.18 87.25) (width 0.35) (layer B.Cu) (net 7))
 (segment (start 73.18 87.25) (end 78.06 82.37) (width 0.35) (layer B.Cu) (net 7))
 (segment (start 78.06 82.37) (end 78.06 76.88) (width 0.35) (layer B.Cu) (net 7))
 (segment (start 78.06 76.88) (end 81.600001 73.339999) (width 0.35) (layer B.Cu) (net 7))
 (segment (start 81.600001 73.339999) (end 82.55 72.39) (width 0.35) (layer B.Cu) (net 7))
 (segment (start 71.82 66.61) (end 79.31 66.61) (width 0.35) (layer B.Cu) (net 8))
 (segment (start 79.31 66.61) (end 82.55 69.85) (width 0.35) (layer B.Cu) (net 8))
 (segment (start 81.600001 66.360001) (end 82.55 67.31) (width 0.35) (layer B.Cu) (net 9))
 (segment (start 73.086 65.1836) (end 80.4236 65.1836) (width 0.35) (layer B.Cu) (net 9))
 (segment (start 71.9724 64.07) (end 73.086 65.1836) (width 0.35) (layer B.Cu) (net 9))
 (segment (start 71.82 64.07) (end 71.9724 64.07) (width 0.25) (layer B.Cu) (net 9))
 (segment (start 80.4236 65.1836) (end 81.600001 66.360001) (width 0.35) (layer B.Cu) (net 9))
 (segment (start 71.942457 55.571728) (end 73.351728 55.571728) (width 0.35) (layer B.Cu) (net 10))
 (segment (start 73.351728 55.571728) (end 82.55 64.77) (width 0.35) (layer B.Cu) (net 10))
 (segment (start 71.942457 53.031728) (end 73.351728 53.031728) (width 0.35) (layer B.Cu) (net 11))
 (segment (start 73.351728 53.031728) (end 82.55 62.23) (width 0.35) (layer B.Cu) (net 11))
 (segment (start 71.82 69.15) (end 76.23 69.15) (width 0.35) (layer B.Cu) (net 1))
 (segment (start 76.23 69.15) (end 71.82 69.15) (width 0.35) (layer B.Cu) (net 1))
 (segment (start 71.82 69.15) (end 71.9 69.23) (width 0.35) (layer B.Cu) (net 1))
 (segment (start 71.9 69.23) (end 76.31 69.23) (width 0.35) (layer B.Cu) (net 1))
 (segment (start 76.31 50.5) (end 76.31 69.23) (width 0.35) (layer F.Cu) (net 1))
 (segment (start 71.82 69.15) (end 76.25 69.26) (width 0.35) (layer B.Cu) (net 1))
 (segment (start 76.311728 50.491728) (end 71.942457 50.491728) (width 0.35) (layer B.Cu) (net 1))
 (segment (start 76.31 50.5) (end 76.311728 50.491728) (width 0.25) (layer B.Cu) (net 1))
 (via (at 76.31 50.5) (size 0.6) (drill 0.4) (layers F.Cu B.Cu) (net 1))
 (via (at 76.31 69.23) (size 0.6) (drill 0.4) (layers F.Cu B.Cu) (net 1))
 (segment (start 76.25 69.26) (end 76.31 69.23) (width 0.25) (layer B.Cu) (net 1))
 (segment (start 69.788996 52.492789) (end 69.788996 56.098996) (width 0.35) (layer B.Cu) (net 1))
 (segment (start 70.601447 51.680338) (end 69.788996 52.492789) (width 0.35) (layer B.Cu) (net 1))
 (segment (start 69.788996 56.098996) (end 74.11 60.42) (width 0.35) (layer B.Cu) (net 1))
 (segment (start 74.11 60.42) (end 74.11 62.51) (width 0.35) (layer B.Cu) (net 1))
 (segment (start 72.535449 62.88139) (end 72.485449 62.83139) (width 0.25) (layer B.Cu) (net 1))
 (segment (start 74.11 62.51) (end 73.73861 62.88139) (width 0.35) (layer B.Cu) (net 1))
 (segment (start 73.73861 62.88139) (end 72.535449 62.88139) (width 0.35) (layer B.Cu) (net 1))
 (segment (start 72.485449 62.83139) (end 71.154551 62.83139) (width 0.25) (layer B.Cu) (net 1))
 (segment (start 70.42899 67.123049) (end 70.47899 67.173049) (width 0.25) (layer B.Cu) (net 1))
 (segment (start 71.154551 62.83139) (end 70.42899 63.556951) (width 0.25) (layer B.Cu) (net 1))
 (segment (start 70.42899 63.556951) (end 70.42899 64.583049) (width 0.25) (layer B.Cu) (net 1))
 (segment (start 70.42899 64.583049) (end 70.47899 64.633049) (width 0.25) (layer B.Cu) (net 1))
 (segment (start 70.47899 64.633049) (end 70.47899 66.046951) (width 0.35) (layer B.Cu) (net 1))
 (segment (start 70.47899 66.046951) (end 70.42899 66.096951) (width 0.25) (layer B.Cu) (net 1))
 (segment (start 70.42899 66.096951) (end 70.42899 67.123049) (width 0.25) (layer B.Cu) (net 1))
 (segment (start 70.47899 67.173049) (end 70.47899 67.96139) (width 0.35) (layer B.Cu) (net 1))
 (segment (start 70.47899 67.96139) (end 71.6676 69.15) (width 0.35) (layer B.Cu) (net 1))
 (segment (start 71.942457 50.491728) (end 73.904179 50.491728) (width 0.25) (layer B.Cu) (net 1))
 (segment (start 73.904179 50.491728) (end 95.91 72.497549) (width 0.35) (layer B.Cu) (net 1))
 (segment (start 95.91 72.497549) (end 95.91 85.75) (width 0.35) (layer B.Cu) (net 1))
 (segment (start 95.91 85.75) (end 99.380001 89.220001) (width 0.35) (layer B.Cu) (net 1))
 (segment (start 99.380001 89.220001) (end 100.33 90.17) (width 0.35) (layer B.Cu) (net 1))
 (segment (start 71.942457 50.491728) (end 71.790057 50.491728) (width 0.25) (layer B.Cu) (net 1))
 (segment (start 71.790057 50.491728) (end 70.601447 51.680338) (width 0.35) (layer B.Cu) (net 1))
 (segment (start 71.6676 69.15) (end 71.82 69.15) (width 0.25) (layer B.Cu) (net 1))
 (segment (start 71.6676 69.15) (end 68.04 72.7776) (width 0.35) (layer B.Cu) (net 1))
 (segment (start 68.04 72.7776) (end 68.04 77.6164) (width 0.35) (layer B.Cu) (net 1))
 (segment (start 68.04 77.6164) (end 71.48 81.0564) (width 0.35) (layer B.Cu) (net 1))
 (segment (start 71.48 81.0564) (end 71.48 82.17) (width 0.35) (layer B.Cu) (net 1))
 (segment (start 68.18 101.24) (end 68.18 85.3176) (width 0.45) (layer B.Cu) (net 1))
 (segment (start 68.18 85.3176) (end 71.3276 82.17) (width 0.45) (layer B.Cu) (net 1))
 (segment (start 71.3276 82.17) (end 71.48 82.17) (width 0.25) (layer B.Cu) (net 1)))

